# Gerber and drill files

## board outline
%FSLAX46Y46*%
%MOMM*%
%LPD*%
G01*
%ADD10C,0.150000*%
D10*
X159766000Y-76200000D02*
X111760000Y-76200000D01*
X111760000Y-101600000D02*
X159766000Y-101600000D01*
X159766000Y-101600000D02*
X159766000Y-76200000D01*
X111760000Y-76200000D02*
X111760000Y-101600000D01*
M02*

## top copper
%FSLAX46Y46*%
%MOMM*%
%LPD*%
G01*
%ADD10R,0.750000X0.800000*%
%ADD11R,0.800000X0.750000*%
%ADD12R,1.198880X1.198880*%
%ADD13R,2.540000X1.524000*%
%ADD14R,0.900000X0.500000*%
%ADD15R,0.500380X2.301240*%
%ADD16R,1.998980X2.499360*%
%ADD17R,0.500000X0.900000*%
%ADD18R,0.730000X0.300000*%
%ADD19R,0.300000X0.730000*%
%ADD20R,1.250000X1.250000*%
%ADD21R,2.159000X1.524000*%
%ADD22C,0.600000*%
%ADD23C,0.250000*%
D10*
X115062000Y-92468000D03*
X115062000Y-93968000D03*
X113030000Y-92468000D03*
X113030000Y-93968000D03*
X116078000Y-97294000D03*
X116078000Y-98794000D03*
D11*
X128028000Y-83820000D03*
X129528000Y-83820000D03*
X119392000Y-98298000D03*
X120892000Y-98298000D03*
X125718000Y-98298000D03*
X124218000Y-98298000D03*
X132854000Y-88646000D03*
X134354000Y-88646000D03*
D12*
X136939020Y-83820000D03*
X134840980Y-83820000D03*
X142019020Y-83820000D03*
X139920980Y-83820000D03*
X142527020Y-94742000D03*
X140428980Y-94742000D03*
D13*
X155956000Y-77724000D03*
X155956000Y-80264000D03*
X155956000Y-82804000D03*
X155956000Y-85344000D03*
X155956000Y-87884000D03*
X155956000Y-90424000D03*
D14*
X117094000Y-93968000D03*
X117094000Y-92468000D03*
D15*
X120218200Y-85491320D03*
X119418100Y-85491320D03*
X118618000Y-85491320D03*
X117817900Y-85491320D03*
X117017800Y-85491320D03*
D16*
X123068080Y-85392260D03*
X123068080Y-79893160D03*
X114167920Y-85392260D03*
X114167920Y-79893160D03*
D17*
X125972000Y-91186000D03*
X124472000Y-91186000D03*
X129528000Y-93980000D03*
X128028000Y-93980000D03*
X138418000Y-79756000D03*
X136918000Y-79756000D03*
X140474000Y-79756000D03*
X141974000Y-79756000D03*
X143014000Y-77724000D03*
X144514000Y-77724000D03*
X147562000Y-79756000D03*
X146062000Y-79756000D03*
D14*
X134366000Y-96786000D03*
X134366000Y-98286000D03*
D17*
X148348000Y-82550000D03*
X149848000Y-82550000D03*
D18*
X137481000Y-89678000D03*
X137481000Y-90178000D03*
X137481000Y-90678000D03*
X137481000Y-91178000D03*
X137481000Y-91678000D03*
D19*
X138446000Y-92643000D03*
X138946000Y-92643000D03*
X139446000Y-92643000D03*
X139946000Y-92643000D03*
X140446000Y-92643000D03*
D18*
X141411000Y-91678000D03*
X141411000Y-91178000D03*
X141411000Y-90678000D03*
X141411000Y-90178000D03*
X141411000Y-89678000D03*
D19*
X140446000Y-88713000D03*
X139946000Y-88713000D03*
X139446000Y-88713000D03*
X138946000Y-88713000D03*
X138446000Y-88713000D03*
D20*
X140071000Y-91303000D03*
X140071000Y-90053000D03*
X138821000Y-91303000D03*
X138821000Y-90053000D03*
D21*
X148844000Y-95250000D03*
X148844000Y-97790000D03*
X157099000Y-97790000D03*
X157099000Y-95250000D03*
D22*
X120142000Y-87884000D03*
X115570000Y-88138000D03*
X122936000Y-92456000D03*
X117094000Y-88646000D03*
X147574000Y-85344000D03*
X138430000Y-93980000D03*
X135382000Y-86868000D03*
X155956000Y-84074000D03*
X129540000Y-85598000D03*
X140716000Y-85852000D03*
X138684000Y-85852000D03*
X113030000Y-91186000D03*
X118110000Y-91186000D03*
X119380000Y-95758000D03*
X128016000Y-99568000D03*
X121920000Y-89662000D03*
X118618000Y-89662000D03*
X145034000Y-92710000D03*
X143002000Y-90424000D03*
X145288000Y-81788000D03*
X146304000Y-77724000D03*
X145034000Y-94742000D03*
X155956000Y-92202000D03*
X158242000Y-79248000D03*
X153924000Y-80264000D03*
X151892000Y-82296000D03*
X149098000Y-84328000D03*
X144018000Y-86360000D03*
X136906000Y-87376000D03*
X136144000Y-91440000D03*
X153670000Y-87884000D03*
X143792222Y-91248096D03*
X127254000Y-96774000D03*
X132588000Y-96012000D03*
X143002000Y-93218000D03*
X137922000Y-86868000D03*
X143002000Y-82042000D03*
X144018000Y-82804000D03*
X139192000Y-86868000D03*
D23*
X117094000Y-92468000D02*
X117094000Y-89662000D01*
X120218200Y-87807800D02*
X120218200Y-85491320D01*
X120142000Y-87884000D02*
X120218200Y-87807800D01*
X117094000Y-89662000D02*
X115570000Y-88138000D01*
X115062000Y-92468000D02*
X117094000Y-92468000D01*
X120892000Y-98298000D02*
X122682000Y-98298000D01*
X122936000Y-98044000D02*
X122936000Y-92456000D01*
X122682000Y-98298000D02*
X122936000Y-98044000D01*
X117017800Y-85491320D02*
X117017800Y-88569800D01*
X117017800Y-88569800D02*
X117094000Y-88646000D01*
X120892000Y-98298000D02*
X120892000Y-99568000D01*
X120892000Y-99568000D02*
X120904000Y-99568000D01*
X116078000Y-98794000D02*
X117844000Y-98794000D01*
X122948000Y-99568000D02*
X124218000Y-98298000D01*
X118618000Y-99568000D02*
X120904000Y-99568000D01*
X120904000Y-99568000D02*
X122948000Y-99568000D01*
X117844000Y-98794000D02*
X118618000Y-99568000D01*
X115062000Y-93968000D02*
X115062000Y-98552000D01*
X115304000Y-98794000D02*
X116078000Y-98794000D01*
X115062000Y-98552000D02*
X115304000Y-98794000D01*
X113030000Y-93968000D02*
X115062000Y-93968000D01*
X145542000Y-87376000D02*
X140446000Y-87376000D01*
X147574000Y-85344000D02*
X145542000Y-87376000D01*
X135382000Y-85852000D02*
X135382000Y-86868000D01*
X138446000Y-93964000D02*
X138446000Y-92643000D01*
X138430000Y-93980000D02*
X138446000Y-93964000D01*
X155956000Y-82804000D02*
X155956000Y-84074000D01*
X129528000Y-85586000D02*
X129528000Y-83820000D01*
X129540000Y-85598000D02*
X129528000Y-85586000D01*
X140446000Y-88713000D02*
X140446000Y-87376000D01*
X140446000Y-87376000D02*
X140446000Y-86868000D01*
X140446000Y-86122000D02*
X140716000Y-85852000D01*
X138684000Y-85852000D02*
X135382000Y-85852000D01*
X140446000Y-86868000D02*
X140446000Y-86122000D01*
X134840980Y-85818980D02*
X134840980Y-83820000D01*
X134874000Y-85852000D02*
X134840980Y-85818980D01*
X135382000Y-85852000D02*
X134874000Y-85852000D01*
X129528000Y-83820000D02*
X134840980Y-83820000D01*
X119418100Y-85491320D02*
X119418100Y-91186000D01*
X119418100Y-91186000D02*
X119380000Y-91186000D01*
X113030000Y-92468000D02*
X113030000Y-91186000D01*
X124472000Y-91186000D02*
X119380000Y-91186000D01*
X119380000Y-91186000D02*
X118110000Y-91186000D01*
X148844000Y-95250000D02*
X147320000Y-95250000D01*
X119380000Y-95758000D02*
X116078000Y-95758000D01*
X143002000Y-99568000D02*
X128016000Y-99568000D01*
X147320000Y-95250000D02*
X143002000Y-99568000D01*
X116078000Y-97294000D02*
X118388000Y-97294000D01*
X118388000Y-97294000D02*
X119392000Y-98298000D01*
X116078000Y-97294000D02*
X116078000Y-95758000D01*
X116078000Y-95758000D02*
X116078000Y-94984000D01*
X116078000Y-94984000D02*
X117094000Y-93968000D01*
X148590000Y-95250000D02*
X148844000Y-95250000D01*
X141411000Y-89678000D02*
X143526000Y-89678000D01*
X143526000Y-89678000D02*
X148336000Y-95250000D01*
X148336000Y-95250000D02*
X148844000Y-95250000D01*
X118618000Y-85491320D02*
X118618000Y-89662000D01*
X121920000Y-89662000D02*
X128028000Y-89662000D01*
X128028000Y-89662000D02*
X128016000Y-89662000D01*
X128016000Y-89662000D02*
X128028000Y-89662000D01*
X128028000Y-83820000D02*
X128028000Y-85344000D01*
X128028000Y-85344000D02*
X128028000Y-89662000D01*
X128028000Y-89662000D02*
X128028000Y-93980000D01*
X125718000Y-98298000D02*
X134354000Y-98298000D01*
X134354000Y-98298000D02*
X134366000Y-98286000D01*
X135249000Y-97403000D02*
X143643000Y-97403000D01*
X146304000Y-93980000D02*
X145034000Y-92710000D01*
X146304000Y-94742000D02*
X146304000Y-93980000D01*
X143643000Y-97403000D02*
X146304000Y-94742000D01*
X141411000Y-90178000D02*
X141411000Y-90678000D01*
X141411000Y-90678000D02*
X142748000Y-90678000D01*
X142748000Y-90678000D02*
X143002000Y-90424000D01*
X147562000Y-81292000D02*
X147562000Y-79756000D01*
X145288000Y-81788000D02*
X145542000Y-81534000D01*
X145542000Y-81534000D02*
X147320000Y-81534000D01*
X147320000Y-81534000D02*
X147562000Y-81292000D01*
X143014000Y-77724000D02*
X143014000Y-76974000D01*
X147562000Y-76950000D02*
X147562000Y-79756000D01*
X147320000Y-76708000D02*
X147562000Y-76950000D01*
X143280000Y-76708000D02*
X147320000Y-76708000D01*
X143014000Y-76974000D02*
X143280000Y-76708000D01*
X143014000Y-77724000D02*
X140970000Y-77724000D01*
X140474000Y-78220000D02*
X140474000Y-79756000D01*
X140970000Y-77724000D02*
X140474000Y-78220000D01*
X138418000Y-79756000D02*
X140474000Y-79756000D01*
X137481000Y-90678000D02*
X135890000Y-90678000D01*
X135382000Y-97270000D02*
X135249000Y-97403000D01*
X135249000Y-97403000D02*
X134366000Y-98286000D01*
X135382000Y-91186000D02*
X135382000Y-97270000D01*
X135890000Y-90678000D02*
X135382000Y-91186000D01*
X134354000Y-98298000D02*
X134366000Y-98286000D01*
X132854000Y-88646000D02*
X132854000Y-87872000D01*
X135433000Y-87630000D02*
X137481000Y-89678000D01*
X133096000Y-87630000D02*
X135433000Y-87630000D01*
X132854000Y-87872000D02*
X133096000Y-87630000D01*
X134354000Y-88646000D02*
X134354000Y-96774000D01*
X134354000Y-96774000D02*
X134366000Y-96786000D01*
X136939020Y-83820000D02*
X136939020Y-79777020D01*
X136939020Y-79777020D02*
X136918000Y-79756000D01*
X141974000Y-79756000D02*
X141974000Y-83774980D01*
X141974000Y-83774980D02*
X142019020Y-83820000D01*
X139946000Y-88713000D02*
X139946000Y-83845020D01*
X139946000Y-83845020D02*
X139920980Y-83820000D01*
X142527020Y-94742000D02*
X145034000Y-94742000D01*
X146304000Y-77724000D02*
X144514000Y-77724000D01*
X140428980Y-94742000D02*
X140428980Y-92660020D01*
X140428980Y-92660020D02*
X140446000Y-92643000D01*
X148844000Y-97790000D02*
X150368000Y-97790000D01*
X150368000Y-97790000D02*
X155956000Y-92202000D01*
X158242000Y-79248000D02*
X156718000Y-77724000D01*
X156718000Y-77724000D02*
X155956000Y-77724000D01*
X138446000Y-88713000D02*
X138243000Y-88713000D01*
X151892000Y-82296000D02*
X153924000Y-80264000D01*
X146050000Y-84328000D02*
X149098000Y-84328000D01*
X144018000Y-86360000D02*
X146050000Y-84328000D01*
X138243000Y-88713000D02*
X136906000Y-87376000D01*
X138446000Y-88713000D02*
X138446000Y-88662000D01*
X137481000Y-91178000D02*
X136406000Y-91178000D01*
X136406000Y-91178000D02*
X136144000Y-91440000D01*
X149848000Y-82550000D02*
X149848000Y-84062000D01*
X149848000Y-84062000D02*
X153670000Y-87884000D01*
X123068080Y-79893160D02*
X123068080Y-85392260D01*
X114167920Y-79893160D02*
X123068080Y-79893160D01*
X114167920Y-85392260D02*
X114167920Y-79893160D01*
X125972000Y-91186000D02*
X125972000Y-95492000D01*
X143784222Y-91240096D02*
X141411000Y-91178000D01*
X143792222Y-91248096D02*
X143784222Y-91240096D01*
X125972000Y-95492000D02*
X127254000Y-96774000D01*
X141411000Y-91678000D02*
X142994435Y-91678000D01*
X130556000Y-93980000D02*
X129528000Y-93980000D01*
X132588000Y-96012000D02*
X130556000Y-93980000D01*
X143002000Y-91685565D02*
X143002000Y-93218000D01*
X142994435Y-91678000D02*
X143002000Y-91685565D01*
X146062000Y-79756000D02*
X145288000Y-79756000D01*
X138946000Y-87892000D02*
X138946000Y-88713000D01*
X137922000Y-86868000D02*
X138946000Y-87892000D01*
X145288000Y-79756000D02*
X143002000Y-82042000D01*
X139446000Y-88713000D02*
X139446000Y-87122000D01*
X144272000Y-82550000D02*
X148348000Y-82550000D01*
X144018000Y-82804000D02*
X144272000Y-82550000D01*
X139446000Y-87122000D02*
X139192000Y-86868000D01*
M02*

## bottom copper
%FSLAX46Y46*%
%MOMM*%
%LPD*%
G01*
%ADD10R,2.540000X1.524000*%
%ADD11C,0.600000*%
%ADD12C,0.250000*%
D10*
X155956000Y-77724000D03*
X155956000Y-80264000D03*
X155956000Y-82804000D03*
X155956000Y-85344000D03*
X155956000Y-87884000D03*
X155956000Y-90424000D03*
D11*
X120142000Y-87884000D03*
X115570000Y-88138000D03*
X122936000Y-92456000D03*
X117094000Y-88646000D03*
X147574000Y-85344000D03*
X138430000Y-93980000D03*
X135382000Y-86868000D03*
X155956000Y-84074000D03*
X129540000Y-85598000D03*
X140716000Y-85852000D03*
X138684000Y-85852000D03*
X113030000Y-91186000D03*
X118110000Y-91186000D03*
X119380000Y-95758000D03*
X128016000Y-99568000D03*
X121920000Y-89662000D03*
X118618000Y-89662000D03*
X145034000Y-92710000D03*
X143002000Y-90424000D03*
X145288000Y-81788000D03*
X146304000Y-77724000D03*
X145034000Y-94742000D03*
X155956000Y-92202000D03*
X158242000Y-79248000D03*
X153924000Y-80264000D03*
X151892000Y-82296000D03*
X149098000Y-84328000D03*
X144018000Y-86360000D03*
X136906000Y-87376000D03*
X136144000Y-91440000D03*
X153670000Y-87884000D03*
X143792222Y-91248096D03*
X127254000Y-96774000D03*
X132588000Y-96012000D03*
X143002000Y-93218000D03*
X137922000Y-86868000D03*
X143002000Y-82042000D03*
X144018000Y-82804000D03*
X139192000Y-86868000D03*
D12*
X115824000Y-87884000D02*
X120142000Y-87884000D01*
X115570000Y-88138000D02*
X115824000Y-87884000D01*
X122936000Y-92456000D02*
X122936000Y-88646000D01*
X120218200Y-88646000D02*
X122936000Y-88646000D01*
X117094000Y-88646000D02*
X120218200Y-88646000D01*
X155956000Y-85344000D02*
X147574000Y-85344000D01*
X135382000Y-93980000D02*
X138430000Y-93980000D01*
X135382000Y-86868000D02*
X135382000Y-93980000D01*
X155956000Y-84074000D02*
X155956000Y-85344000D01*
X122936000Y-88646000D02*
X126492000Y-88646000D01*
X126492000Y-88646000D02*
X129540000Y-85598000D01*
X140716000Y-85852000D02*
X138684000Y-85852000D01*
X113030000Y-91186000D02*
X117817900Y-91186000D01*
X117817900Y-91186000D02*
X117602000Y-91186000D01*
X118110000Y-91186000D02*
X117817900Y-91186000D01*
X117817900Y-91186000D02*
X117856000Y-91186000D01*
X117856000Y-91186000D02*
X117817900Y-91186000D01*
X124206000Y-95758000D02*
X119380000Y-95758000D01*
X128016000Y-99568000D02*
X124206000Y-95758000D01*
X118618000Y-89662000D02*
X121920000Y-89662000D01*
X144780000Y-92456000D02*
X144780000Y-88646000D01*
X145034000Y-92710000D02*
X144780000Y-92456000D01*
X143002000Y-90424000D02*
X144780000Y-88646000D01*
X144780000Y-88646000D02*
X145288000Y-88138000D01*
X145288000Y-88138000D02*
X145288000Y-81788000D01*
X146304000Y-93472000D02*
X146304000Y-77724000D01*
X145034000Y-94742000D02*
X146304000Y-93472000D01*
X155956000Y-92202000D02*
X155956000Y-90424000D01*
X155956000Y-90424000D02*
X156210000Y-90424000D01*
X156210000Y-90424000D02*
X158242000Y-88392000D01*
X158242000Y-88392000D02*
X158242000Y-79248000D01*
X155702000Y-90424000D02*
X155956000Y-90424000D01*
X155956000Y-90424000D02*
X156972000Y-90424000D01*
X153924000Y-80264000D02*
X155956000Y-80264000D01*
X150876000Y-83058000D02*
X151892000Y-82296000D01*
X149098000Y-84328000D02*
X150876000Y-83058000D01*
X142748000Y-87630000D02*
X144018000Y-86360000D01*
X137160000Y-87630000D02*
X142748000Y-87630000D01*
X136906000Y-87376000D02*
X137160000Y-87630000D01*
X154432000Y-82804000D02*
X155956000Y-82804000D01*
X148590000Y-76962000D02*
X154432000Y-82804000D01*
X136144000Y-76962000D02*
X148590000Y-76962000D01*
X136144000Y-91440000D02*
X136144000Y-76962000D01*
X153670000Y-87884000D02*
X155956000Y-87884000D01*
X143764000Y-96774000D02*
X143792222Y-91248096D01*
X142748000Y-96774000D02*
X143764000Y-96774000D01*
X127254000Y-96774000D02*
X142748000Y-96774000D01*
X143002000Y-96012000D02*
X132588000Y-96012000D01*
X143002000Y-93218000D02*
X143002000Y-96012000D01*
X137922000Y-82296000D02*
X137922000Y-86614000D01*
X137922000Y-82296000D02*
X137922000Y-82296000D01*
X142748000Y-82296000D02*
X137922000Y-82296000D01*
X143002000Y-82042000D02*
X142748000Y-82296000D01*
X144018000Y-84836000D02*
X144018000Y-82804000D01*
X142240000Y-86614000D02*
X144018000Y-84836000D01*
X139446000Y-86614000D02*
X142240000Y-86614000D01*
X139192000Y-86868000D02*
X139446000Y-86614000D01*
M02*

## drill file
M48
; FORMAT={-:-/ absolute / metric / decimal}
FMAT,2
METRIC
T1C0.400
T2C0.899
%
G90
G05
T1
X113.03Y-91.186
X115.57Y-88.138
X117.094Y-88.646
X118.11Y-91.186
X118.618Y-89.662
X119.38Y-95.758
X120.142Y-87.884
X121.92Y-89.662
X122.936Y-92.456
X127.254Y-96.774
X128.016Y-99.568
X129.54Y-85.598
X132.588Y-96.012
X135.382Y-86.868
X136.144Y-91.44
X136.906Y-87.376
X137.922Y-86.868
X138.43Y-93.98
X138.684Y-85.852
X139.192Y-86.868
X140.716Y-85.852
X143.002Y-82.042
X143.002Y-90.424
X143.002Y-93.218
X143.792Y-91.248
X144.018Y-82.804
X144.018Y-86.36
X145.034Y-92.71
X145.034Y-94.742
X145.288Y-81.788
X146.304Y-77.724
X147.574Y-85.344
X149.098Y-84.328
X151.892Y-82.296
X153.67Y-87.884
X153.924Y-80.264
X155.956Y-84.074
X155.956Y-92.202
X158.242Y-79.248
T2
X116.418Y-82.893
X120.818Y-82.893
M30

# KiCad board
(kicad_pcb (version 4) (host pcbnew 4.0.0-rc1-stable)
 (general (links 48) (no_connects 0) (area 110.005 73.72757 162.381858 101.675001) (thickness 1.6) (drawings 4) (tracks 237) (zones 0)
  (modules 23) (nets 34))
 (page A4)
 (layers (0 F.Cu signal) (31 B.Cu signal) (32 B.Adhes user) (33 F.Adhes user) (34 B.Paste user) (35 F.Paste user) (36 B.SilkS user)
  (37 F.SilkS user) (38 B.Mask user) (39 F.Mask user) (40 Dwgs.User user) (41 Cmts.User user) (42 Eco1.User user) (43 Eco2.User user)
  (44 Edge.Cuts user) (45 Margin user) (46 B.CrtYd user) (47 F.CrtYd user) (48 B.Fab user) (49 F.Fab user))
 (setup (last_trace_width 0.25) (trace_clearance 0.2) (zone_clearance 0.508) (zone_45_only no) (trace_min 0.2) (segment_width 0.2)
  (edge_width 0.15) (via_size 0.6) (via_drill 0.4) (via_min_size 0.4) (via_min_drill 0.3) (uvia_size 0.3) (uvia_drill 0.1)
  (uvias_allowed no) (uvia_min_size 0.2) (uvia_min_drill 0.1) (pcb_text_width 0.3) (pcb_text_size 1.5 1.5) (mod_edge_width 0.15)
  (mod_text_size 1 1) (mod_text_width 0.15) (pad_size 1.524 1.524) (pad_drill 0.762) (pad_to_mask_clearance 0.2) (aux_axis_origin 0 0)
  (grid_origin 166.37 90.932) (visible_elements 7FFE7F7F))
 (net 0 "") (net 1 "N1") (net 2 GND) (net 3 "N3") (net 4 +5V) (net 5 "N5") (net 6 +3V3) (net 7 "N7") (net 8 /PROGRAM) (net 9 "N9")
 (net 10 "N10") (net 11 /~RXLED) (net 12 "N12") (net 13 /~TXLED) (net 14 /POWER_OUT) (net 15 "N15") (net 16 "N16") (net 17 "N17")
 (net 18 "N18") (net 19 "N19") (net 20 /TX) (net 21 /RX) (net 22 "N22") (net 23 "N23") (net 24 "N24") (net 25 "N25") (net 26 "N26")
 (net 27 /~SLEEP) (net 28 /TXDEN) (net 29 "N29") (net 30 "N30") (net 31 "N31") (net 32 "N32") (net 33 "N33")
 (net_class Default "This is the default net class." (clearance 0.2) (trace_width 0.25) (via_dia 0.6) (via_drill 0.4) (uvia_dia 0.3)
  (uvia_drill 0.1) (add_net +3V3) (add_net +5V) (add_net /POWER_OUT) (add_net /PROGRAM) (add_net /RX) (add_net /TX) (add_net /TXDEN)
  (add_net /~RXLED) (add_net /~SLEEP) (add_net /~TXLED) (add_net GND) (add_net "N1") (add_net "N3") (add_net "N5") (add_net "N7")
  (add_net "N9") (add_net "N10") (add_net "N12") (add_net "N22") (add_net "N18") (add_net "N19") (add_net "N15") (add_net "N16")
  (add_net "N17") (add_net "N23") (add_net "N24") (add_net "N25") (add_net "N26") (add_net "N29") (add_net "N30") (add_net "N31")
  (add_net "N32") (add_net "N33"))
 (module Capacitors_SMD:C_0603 (layer F.Cu) (at 115.062 93.218 270)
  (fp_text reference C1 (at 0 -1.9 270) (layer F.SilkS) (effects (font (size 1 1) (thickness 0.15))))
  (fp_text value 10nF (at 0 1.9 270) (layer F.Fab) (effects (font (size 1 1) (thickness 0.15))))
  (pad 1 smd rect (at -0.75 0 270) (size 0.8 0.75) (layers F.Cu F.Paste F.Mask) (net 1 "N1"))
  (pad 2 smd rect (at 0.75 0 270) (size 0.8 0.75) (layers F.Cu F.Paste F.Mask) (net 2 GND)))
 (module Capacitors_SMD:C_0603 (layer F.Cu) (at 113.03 93.218 270)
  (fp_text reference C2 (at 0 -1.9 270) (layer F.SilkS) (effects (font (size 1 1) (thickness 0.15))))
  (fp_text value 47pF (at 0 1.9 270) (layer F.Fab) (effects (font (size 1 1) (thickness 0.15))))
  (pad 1 smd rect (at -0.75 0 270) (size 0.8 0.75) (layers F.Cu F.Paste F.Mask) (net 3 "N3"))
  (pad 2 smd rect (at 0.75 0 270) (size 0.8 0.75) (layers F.Cu F.Paste F.Mask) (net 2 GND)))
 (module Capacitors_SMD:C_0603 (layer F.Cu) (at 116.078 98.044 270)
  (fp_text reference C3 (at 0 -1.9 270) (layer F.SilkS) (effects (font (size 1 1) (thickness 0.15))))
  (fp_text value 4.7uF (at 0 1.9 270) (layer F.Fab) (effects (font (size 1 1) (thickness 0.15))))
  (pad 1 smd rect (at -0.75 0 270) (size 0.8 0.75) (layers F.Cu F.Paste F.Mask) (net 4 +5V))
  (pad 2 smd rect (at 0.75 0 270) (size 0.8 0.75) (layers F.Cu F.Paste F.Mask) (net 2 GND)))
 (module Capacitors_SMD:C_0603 (layer F.Cu) (at 128.778 83.82)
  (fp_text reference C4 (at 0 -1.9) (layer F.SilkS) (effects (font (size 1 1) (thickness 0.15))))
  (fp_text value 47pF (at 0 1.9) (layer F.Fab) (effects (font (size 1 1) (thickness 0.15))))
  (pad 1 smd rect (at -0.75 0) (size 0.8 0.75) (layers F.Cu F.Paste F.Mask) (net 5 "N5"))
  (pad 2 smd rect (at 0.75 0) (size 0.8 0.75) (layers F.Cu F.Paste F.Mask) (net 2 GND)))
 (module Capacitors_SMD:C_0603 (layer F.Cu) (at 120.142 98.298)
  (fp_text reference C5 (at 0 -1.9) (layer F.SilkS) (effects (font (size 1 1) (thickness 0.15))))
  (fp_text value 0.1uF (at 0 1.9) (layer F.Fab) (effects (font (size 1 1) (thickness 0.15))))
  (pad 1 smd rect (at -0.75 0) (size 0.8 0.75) (layers F.Cu F.Paste F.Mask) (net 4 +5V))
  (pad 2 smd rect (at 0.75 0) (size 0.8 0.75) (layers F.Cu F.Paste F.Mask) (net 2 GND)))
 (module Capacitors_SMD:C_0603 (layer F.Cu) (at 124.968 98.298 180)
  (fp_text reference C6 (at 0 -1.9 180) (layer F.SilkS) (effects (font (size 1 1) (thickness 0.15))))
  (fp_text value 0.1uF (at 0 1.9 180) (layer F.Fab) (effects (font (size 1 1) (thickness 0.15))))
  (pad 1 smd rect (at -0.75 0 180) (size 0.8 0.75) (layers F.Cu F.Paste F.Mask) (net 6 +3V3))
  (pad 2 smd rect (at 0.75 0 180) (size 0.8 0.75) (layers F.Cu F.Paste F.Mask) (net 2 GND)))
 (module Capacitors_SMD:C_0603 (layer F.Cu) (at 133.604 88.646)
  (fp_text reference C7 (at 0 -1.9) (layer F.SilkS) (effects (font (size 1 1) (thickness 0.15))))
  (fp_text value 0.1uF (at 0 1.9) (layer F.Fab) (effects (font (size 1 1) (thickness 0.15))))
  (pad 1 smd rect (at -0.75 0) (size 0.8 0.75) (layers F.Cu F.Paste F.Mask) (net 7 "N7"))
  (pad 2 smd rect (at 0.75 0) (size 0.8 0.75) (layers F.Cu F.Paste F.Mask) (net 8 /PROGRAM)))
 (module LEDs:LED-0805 (layer F.Cu) (at 135.89 83.82)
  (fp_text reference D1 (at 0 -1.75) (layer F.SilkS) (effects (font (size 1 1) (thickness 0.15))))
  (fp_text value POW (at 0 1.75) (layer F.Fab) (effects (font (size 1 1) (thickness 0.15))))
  (pad 2 smd rect (at 1.04902 0 180) (size 1.19888 1.19888) (layers F.Cu F.Paste F.Mask) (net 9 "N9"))
  (pad 1 smd rect (at -1.04902 0 180) (size 1.19888 1.19888) (layers F.Cu F.Paste F.Mask) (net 2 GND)))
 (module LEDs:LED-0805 (layer F.Cu) (at 140.97 83.82)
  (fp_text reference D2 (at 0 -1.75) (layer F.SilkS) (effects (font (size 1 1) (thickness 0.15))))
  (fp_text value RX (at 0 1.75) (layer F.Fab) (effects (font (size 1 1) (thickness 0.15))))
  (pad 2 smd rect (at 1.04902 0 180) (size 1.19888 1.19888) (layers F.Cu F.Paste F.Mask) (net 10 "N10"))
  (pad 1 smd rect (at -1.04902 0 180) (size 1.19888 1.19888) (layers F.Cu F.Paste F.Mask) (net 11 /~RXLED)))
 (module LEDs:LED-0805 (layer F.Cu) (at 141.478 94.742)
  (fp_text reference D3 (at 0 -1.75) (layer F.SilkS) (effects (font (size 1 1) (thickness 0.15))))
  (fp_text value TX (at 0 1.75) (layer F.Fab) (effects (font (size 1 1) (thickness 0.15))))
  (pad 2 smd rect (at 1.04902 0 180) (size 1.19888 1.19888) (layers F.Cu F.Paste F.Mask) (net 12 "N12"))
  (pad 1 smd rect (at -1.04902 0 180) (size 1.19888 1.19888) (layers F.Cu F.Paste F.Mask) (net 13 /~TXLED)))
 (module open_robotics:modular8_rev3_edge (layer F.Cu) (at 155.956 82.804 270)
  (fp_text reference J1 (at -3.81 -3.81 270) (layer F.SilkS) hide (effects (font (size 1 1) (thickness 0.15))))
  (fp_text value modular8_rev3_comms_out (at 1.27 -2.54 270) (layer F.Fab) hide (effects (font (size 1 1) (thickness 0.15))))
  (pad 1 smd rect (at -5.08 0 270) (size 1.524 2.54) (layers F.Cu F.Paste F.Mask) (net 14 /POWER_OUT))
  (pad 3 smd rect (at -2.54 0 270) (size 1.524 2.54) (layers F.Cu F.Paste F.Mask) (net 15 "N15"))
  (pad 5 smd rect (at 0 0 270) (size 1.524 2.54) (layers F.Cu F.Paste F.Mask) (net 2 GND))
  (pad 7 smd rect (at 2.54 0 270) (size 1.524 2.54) (layers F.Cu F.Paste F.Mask) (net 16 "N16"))
  (pad 9 smd rect (at 5.08 0 270) (size 1.524 2.54) (layers F.Cu F.Paste F.Mask) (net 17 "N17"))
  (pad 11 smd rect (at 7.62 0 270) (size 1.524 2.54) (layers F.Cu F.Paste F.Mask) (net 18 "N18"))
  (pad 2 smd rect (at -5.08 0 270) (size 1.524 2.54) (layers B.Cu F.Paste F.Mask) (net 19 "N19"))
  (pad 4 smd rect (at -2.54 0 270) (size 1.524 2.54) (layers B.Cu F.Paste F.Mask) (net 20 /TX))
  (pad 6 smd rect (at 0 0 270) (size 1.524 2.54) (layers B.Cu F.Paste F.Mask) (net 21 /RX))
  (pad 8 smd rect (at 2.54 0 270) (size 1.524 2.54) (layers B.Cu F.Paste F.Mask) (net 2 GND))
  (pad 10 smd rect (at 5.08 0 270) (size 1.524 2.54) (layers B.Cu F.Paste F.Mask) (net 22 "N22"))
  (pad 12 smd rect (at 7.62 0 270) (size 1.524 2.54) (layers B.Cu F.Paste F.Mask) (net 14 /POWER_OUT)))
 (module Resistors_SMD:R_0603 (layer F.Cu) (at 117.094 93.218 90)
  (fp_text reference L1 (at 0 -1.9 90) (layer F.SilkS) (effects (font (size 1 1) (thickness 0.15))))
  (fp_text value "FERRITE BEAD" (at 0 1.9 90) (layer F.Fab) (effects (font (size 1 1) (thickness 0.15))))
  (pad 1 smd rect (at -0.75 0 90) (size 0.5 0.9) (layers F.Cu F.Paste F.Mask) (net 4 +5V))
  (pad 2 smd rect (at 0.75 0 90) (size 0.5 0.9) (layers F.Cu F.Paste F.Mask) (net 1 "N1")))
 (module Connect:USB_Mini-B (layer F.Cu) (at 118.618 82.042 270)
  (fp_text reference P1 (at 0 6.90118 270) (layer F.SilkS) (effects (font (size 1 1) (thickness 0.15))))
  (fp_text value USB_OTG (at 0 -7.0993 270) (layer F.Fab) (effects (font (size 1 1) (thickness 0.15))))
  (pad 1 smd rect (at 3.44932 -1.6002 270) (size 2.30124 0.50038) (layers F.Cu F.Paste F.Mask) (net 1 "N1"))
  (pad 2 smd rect (at 3.44932 -0.8001 270) (size 2.30124 0.50038) (layers F.Cu F.Paste F.Mask) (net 3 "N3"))
  (pad 3 smd rect (at 3.44932 0 270) (size 2.30124 0.50038) (layers F.Cu F.Paste F.Mask) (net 5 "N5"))
  (pad 4 smd rect (at 3.44932 0.8001 270) (size 2.30124 0.50038) (layers F.Cu F.Paste F.Mask) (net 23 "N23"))
  (pad 5 smd rect (at 3.44932 1.6002 270) (size 2.30124 0.50038) (layers F.Cu F.Paste F.Mask) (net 2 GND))
  (pad 6 smd rect (at 3.35026 -4.45008 270) (size 2.49936 1.99898) (layers F.Cu F.Paste F.Mask) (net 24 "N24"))
  (pad 6 smd rect (at -2.14884 -4.45008 270) (size 2.49936 1.99898) (layers F.Cu F.Paste F.Mask) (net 24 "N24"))
  (pad 6 smd rect (at 3.35026 4.45008 270) (size 2.49936 1.99898) (layers F.Cu F.Paste F.Mask) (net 24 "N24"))
  (pad 6 smd rect (at -2.14884 4.45008 270) (size 2.49936 1.99898) (layers F.Cu F.Paste F.Mask) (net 24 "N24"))
  (pad "" np_thru_hole circle (at 0.8509 -2.19964 270) (size 0.89916 0.89916) (drill 0.89916) (layers *.Cu *.Mask F.SilkS))
  (pad "" np_thru_hole circle (at 0.8509 2.19964 270) (size 0.89916 0.89916) (drill 0.89916) (layers *.Cu *.Mask F.SilkS)))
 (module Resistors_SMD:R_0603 (layer F.Cu) (at 125.222 91.186 180)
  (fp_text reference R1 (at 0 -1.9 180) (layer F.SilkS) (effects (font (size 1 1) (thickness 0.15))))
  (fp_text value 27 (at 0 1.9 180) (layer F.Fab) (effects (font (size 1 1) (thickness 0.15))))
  (pad 1 smd rect (at -0.75 0 180) (size 0.5 0.9) (layers F.Cu F.Paste F.Mask) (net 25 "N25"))
  (pad 2 smd rect (at 0.75 0 180) (size 0.5 0.9) (layers F.Cu F.Paste F.Mask) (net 3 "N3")))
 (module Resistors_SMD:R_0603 (layer F.Cu) (at 128.778 93.98 180)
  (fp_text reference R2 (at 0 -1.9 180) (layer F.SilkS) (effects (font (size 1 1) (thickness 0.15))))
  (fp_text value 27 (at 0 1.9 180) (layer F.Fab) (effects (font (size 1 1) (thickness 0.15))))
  (pad 1 smd rect (at -0.75 0 180) (size 0.5 0.9) (layers F.Cu F.Paste F.Mask) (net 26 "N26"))
  (pad 2 smd rect (at 0.75 0 180) (size 0.5 0.9) (layers F.Cu F.Paste F.Mask) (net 5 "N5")))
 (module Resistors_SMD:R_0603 (layer F.Cu) (at 137.668 79.756 180)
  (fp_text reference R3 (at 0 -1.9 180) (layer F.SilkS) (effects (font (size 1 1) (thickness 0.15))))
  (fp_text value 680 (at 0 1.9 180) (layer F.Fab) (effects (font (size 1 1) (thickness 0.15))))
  (pad 1 smd rect (at -0.75 0 180) (size 0.5 0.9) (layers F.Cu F.Paste F.Mask) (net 6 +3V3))
  (pad 2 smd rect (at 0.75 0 180) (size 0.5 0.9) (layers F.Cu F.Paste F.Mask) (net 9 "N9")))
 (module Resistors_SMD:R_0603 (layer F.Cu) (at 141.224 79.756)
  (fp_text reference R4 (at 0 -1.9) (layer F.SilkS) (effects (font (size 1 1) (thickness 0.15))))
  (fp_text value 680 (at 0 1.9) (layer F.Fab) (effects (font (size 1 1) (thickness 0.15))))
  (pad 1 smd rect (at -0.75 0) (size 0.5 0.9) (layers F.Cu F.Paste F.Mask) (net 6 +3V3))
  (pad 2 smd rect (at 0.75 0) (size 0.5 0.9) (layers F.Cu F.Paste F.Mask) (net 10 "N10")))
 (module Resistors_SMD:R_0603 (layer F.Cu) (at 143.764 77.724)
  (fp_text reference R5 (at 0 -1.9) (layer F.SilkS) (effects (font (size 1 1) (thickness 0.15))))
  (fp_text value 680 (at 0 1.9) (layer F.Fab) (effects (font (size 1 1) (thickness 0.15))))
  (pad 1 smd rect (at -0.75 0) (size 0.5 0.9) (layers F.Cu F.Paste F.Mask) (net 6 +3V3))
  (pad 2 smd rect (at 0.75 0) (size 0.5 0.9) (layers F.Cu F.Paste F.Mask) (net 12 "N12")))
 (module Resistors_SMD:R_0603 (layer F.Cu) (at 146.812 79.756 180)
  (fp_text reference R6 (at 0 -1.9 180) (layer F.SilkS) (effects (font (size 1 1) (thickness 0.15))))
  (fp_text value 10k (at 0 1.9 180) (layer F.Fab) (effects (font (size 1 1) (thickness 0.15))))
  (pad 1 smd rect (at -0.75 0 180) (size 0.5 0.9) (layers F.Cu F.Paste F.Mask) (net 6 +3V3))
  (pad 2 smd rect (at 0.75 0 180) (size 0.5 0.9) (layers F.Cu F.Paste F.Mask) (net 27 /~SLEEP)))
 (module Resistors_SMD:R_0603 (layer F.Cu) (at 134.366 97.536 270)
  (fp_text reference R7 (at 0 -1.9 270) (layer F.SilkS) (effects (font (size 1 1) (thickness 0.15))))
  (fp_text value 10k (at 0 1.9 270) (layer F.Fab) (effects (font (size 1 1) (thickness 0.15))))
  (pad 1 smd rect (at -0.75 0 270) (size 0.5 0.9) (layers F.Cu F.Paste F.Mask) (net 8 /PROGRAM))
  (pad 2 smd rect (at 0.75 0 270) (size 0.5 0.9) (layers F.Cu F.Paste F.Mask) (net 6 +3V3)))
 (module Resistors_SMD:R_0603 (layer F.Cu) (at 149.098 82.55)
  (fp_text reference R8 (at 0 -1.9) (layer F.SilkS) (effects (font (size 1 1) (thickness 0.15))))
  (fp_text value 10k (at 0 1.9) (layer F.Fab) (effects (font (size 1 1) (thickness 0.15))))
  (pad 1 smd rect (at -0.75 0) (size 0.5 0.9) (layers F.Cu F.Paste F.Mask) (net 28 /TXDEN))
  (pad 2 smd rect (at 0.75 0) (size 0.5 0.9) (layers F.Cu F.Paste F.Mask) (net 22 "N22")))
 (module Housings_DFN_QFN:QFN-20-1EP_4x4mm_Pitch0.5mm (layer F.Cu) (at 139.446 90.678)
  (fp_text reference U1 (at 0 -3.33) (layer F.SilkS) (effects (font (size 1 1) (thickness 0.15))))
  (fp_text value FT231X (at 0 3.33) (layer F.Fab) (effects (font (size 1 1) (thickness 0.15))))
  (pad 1 smd rect (at -1.965 -1) (size 0.73 0.3) (layers F.Cu F.Paste F.Mask) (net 7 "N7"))
  (pad 2 smd rect (at -1.965 -0.5) (size 0.73 0.3) (layers F.Cu F.Paste F.Mask) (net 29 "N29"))
  (pad 3 smd rect (at -1.965 0) (size 0.73 0.3) (layers F.Cu F.Paste F.Mask) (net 6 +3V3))
  (pad 4 smd rect (at -1.965 0.5) (size 0.73 0.3) (layers F.Cu F.Paste F.Mask) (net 21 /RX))
  (pad 5 smd rect (at -1.965 1) (size 0.73 0.3) (layers F.Cu F.Paste F.Mask) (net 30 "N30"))
  (pad 6 smd rect (at -1 1.965 90) (size 0.73 0.3) (layers F.Cu F.Paste F.Mask) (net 2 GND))
  (pad 7 smd rect (at -0.5 1.965 90) (size 0.73 0.3) (layers F.Cu F.Paste F.Mask) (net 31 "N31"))
  (pad 8 smd rect (at 0 1.965 90) (size 0.73 0.3) (layers F.Cu F.Paste F.Mask) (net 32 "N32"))
  (pad 9 smd rect (at 0.5 1.965 90) (size 0.73 0.3) (layers F.Cu F.Paste F.Mask) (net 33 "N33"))
  (pad 10 smd rect (at 1 1.965 90) (size 0.73 0.3) (layers F.Cu F.Paste F.Mask) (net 13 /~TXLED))
  (pad 11 smd rect (at 1.965 1) (size 0.73 0.3) (layers F.Cu F.Paste F.Mask) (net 26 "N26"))
  (pad 12 smd rect (at 1.965 0.5) (size 0.73 0.3) (layers F.Cu F.Paste F.Mask) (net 25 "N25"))
  (pad 13 smd rect (at 1.965 0) (size 0.73 0.3) (layers F.Cu F.Paste F.Mask) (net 6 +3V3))
  (pad 14 smd rect (at 1.965 -0.5) (size 0.73 0.3) (layers F.Cu F.Paste F.Mask) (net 6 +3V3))
  (pad 15 smd rect (at 1.965 -1) (size 0.73 0.3) (layers F.Cu F.Paste F.Mask) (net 4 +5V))
  (pad 16 smd rect (at 1 -1.965 90) (size 0.73 0.3) (layers F.Cu F.Paste F.Mask) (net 2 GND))
  (pad 17 smd rect (at 0.5 -1.965 90) (size 0.73 0.3) (layers F.Cu F.Paste F.Mask) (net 11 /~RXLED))
  (pad 18 smd rect (at 0 -1.965 90) (size 0.73 0.3) (layers F.Cu F.Paste F.Mask) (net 28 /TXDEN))
  (pad 19 smd rect (at -0.5 -1.965 90) (size 0.73 0.3) (layers F.Cu F.Paste F.Mask) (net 27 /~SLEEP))
  (pad 20 smd rect (at -1 -1.965 90) (size 0.73 0.3) (layers F.Cu F.Paste F.Mask) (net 20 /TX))
  (pad 21 smd rect (at 0.625 0.625) (size 1.25 1.25) (layers F.Cu F.Paste F.Mask) (solder_paste_margin_ratio -0.2))
  (pad 21 smd rect (at 0.625 -0.625) (size 1.25 1.25) (layers F.Cu F.Paste F.Mask) (solder_paste_margin_ratio -0.2))
  (pad 21 smd rect (at -0.625 0.625) (size 1.25 1.25) (layers F.Cu F.Paste F.Mask) (solder_paste_margin_ratio -0.2))
  (pad 21 smd rect (at -0.625 -0.625) (size 1.25 1.25) (layers F.Cu F.Paste F.Mask) (solder_paste_margin_ratio -0.2)))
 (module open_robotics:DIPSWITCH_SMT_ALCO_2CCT (layer F.Cu) (at 148.844 95.25)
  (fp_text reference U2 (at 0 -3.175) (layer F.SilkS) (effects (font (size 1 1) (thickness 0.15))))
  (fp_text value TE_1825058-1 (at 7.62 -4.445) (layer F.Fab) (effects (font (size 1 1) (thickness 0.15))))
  (pad 1 smd rect (at 0 0) (size 2.159 1.524) (layers F.Cu F.Paste F.Mask) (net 4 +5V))
  (pad 2 smd rect (at 0 2.54) (size 2.159 1.524) (layers F.Cu F.Paste F.Mask) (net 14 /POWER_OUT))
  (pad 3 smd rect (at 8.255 2.54) (size 2.159 1.524) (layers F.Cu F.Paste F.Mask))
  (pad 4 smd rect (at 8.255 0) (size 2.159 1.524) (layers F.Cu F.Paste F.Mask)))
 (gr_line (start 159.766 76.2) (end 111.76 76.2) (angle 90) (layer Edge.Cuts) (width 0.15))
 (gr_line (start 111.76 101.6) (end 159.766 101.6) (angle 90) (layer Edge.Cuts) (width 0.15))
 (gr_line (start 159.766 101.6) (end 159.766 76.2) (angle 90) (layer Edge.Cuts) (width 0.15))
 (gr_line (start 111.76 76.2) (end 111.76 101.6) (angle 90) (layer Edge.Cuts) (width 0.15))
 (segment (start 117.094 92.468) (end 117.094 89.662) (width 0.25) (layer F.Cu) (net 1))
 (segment (start 120.2182 87.8078) (end 120.2182 85.49132) (width 0.25) (layer F.Cu) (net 1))
 (segment (start 120.142 87.884) (end 120.2182 87.8078) (width 0.25) (layer F.Cu) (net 1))
 (via (at 120.142 87.884) (size 0.6) (drill 0.4) (layers F.Cu B.Cu) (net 1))
 (segment (start 115.824 87.884) (end 120.142 87.884) (width 0.25) (layer B.Cu) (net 1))
 (segment (start 115.57 88.138) (end 115.824 87.884) (width 0.25) (layer B.Cu) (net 1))
 (via (at 115.57 88.138) (size 0.6) (drill 0.4) (layers F.Cu B.Cu) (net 1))
 (segment (start 117.094 89.662) (end 115.57 88.138) (width 0.25) (layer F.Cu) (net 1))
 (segment (start 115.062 92.468) (end 117.094 92.468) (width 0.25) (layer F.Cu) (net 1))
 (segment (start 120.892 98.298) (end 122.682 98.298) (width 0.25) (layer F.Cu) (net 2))
 (segment (start 122.936 92.456) (end 122.936 88.646) (width 0.25) (layer B.Cu) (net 2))
 (via (at 122.936 92.456) (size 0.6) (drill 0.4) (layers F.Cu B.Cu) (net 2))
 (segment (start 122.936 98.044) (end 122.936 92.456) (width 0.25) (layer F.Cu) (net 2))
 (segment (start 122.682 98.298) (end 122.936 98.044) (width 0.25) (layer F.Cu) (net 2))
 (segment (start 117.0178 85.49132) (end 117.0178 88.5698) (width 0.25) (layer F.Cu) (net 2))
 (segment (start 120.2182 88.646) (end 122.936 88.646) (width 0.25) (layer B.Cu) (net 2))
 (segment (start 117.0178 88.5698) (end 117.094 88.646) (width 0.25) (layer F.Cu) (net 2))
 (via (at 117.094 88.646) (size 0.6) (drill 0.4) (layers F.Cu B.Cu) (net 2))
 (segment (start 117.094 88.646) (end 120.2182 88.646) (width 0.25) (layer B.Cu) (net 2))
 (segment (start 120.892 98.298) (end 120.892 99.568) (width 0.25) (layer F.Cu) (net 2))
 (segment (start 120.892 99.568) (end 120.904 99.568) (width 0.25) (layer F.Cu) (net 2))
 (segment (start 116.078 98.794) (end 117.844 98.794) (width 0.25) (layer F.Cu) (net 2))
 (segment (start 122.948 99.568) (end 124.218 98.298) (width 0.25) (layer F.Cu) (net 2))
 (segment (start 118.618 99.568) (end 120.904 99.568) (width 0.25) (layer F.Cu) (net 2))
 (segment (start 120.904 99.568) (end 122.948 99.568) (width 0.25) (layer F.Cu) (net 2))
 (segment (start 117.844 98.794) (end 118.618 99.568) (width 0.25) (layer F.Cu) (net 2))
 (segment (start 115.062 93.968) (end 115.062 98.552) (width 0.25) (layer F.Cu) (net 2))
 (segment (start 115.304 98.794) (end 116.078 98.794) (width 0.25) (layer F.Cu) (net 2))
 (segment (start 115.062 98.552) (end 115.304 98.794) (width 0.25) (layer F.Cu) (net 2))
 (segment (start 113.03 93.968) (end 115.062 93.968) (width 0.25) (layer F.Cu) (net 2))
 (segment (start 155.956 85.344) (end 147.574 85.344) (width 0.25) (layer B.Cu) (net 2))
 (segment (start 145.542 87.376) (end 140.446 87.376) (width 0.25) (layer F.Cu) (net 2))
 (segment (start 147.574 85.344) (end 145.542 87.376) (width 0.25) (layer F.Cu) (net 2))
 (via (at 147.574 85.344) (size 0.6) (drill 0.4) (layers F.Cu B.Cu) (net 2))
 (segment (start 135.382 85.852) (end 135.382 86.868) (width 0.25) (layer F.Cu) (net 2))
 (segment (start 138.446 93.964) (end 138.446 92.643) (width 0.25) (layer F.Cu) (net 2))
 (segment (start 138.43 93.98) (end 138.446 93.964) (width 0.25) (layer F.Cu) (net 2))
 (via (at 138.43 93.98) (size 0.6) (drill 0.4) (layers F.Cu B.Cu) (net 2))
 (segment (start 135.382 93.98) (end 138.43 93.98) (width 0.25) (layer B.Cu) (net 2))
 (segment (start 135.382 86.868) (end 135.382 93.98) (width 0.25) (layer B.Cu) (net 2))
 (via (at 135.382 86.868) (size 0.6) (drill 0.4) (layers F.Cu B.Cu) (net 2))
 (segment (start 155.956 82.804) (end 155.956 84.074) (width 0.25) (layer F.Cu) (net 2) (status 10))
 (segment (start 155.956 84.074) (end 155.956 85.344) (width 0.25) (layer B.Cu) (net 2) (status 20))
 (via (at 155.956 84.074) (size 0.6) (drill 0.4) (layers F.Cu B.Cu) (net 2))
 (segment (start 122.936 88.646) (end 126.492 88.646) (width 0.25) (layer B.Cu) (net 2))
 (segment (start 129.528 85.586) (end 129.528 83.82) (width 0.25) (layer F.Cu) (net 2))
 (segment (start 129.54 85.598) (end 129.528 85.586) (width 0.25) (layer F.Cu) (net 2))
 (via (at 129.54 85.598) (size 0.6) (drill 0.4) (layers F.Cu B.Cu) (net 2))
 (segment (start 126.492 88.646) (end 129.54 85.598) (width 0.25) (layer B.Cu) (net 2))
 (segment (start 140.446 88.713) (end 140.446 87.376) (width 0.25) (layer F.Cu) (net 2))
 (segment (start 140.446 87.376) (end 140.446 86.868) (width 0.25) (layer F.Cu) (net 2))
 (segment (start 140.446 86.122) (end 140.716 85.852) (width 0.25) (layer F.Cu) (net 2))
 (via (at 140.716 85.852) (size 0.6) (drill 0.4) (layers F.Cu B.Cu) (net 2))
 (segment (start 140.716 85.852) (end 138.684 85.852) (width 0.25) (layer B.Cu) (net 2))
 (via (at 138.684 85.852) (size 0.6) (drill 0.4) (layers F.Cu B.Cu) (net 2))
 (segment (start 138.684 85.852) (end 135.382 85.852) (width 0.25) (layer F.Cu) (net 2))
 (segment (start 140.446 86.868) (end 140.446 86.122) (width 0.25) (layer F.Cu) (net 2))
 (segment (start 134.84098 85.81898) (end 134.84098 83.82) (width 0.25) (layer F.Cu) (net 2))
 (segment (start 134.874 85.852) (end 134.84098 85.81898) (width 0.25) (layer F.Cu) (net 2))
 (segment (start 135.382 85.852) (end 134.874 85.852) (width 0.25) (layer F.Cu) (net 2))
 (segment (start 129.528 83.82) (end 134.84098 83.82) (width 0.25) (layer F.Cu) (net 2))
 (segment (start 119.4181 85.49132) (end 119.4181 91.186) (width 0.25) (layer F.Cu) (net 3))
 (segment (start 119.4181 91.186) (end 119.38 91.186) (width 0.25) (layer F.Cu) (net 3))
 (segment (start 113.03 92.468) (end 113.03 91.186) (width 0.25) (layer F.Cu) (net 3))
 (segment (start 113.03 91.186) (end 117.8179 91.186) (width 0.25) (layer B.Cu) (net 3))
 (via (at 113.03 91.186) (size 0.6) (drill 0.4) (layers F.Cu B.Cu) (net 3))
 (segment (start 117.8179 91.186) (end 117.602 91.186) (width 0.25) (layer B.Cu) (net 3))
 (segment (start 124.472 91.186) (end 119.38 91.186) (width 0.25) (layer F.Cu) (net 3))
 (segment (start 119.38 91.186) (end 118.11 91.186) (width 0.25) (layer F.Cu) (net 3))
 (segment (start 118.11 91.186) (end 117.8179 91.186) (width 0.25) (layer B.Cu) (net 3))
 (via (at 118.11 91.186) (size 0.6) (drill 0.4) (layers F.Cu B.Cu) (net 3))
 (segment (start 117.8179 91.186) (end 117.856 91.186) (width 0.25) (layer B.Cu) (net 3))
 (segment (start 117.856 91.186) (end 117.8179 91.186) (width 0.25) (layer B.Cu) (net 3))
 (segment (start 148.844 95.25) (end 147.32 95.25) (width 0.25) (layer F.Cu) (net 4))
 (segment (start 119.38 95.758) (end 116.078 95.758) (width 0.25) (layer F.Cu) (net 4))
 (via (at 119.38 95.758) (size 0.6) (drill 0.4) (layers F.Cu B.Cu) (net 4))
 (segment (start 124.206 95.758) (end 119.38 95.758) (width 0.25) (layer B.Cu) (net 4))
 (segment (start 128.016 99.568) (end 124.206 95.758) (width 0.25) (layer B.Cu) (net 4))
 (via (at 128.016 99.568) (size 0.6) (drill 0.4) (layers F.Cu B.Cu) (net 4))
 (segment (start 143.002 99.568) (end 128.016 99.568) (width 0.25) (layer F.Cu) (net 4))
 (segment (start 147.32 95.25) (end 143.002 99.568) (width 0.25) (layer F.Cu) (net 4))
 (segment (start 116.078 97.294) (end 118.388 97.294) (width 0.25) (layer F.Cu) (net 4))
 (segment (start 118.388 97.294) (end 119.392 98.298) (width 0.25) (layer F.Cu) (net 4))
 (segment (start 116.078 97.294) (end 116.078 95.758) (width 0.25) (layer F.Cu) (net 4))
 (segment (start 116.078 95.758) (end 116.078 94.984) (width 0.25) (layer F.Cu) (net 4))
 (segment (start 116.078 94.984) (end 117.094 93.968) (width 0.25) (layer F.Cu) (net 4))
 (segment (start 148.59 95.25) (end 148.844 95.25) (width 0.25) (layer F.Cu) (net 4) (status 30))
 (segment (start 141.411 89.678) (end 143.526 89.678) (width 0.25) (layer F.Cu) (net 4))
 (segment (start 143.526 89.678) (end 148.336 95.25) (width 0.25) (layer F.Cu) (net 4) (status 20))
 (segment (start 148.336 95.25) (end 148.844 95.25) (width 0.25) (layer F.Cu) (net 4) (status 30))
 (segment (start 118.618 85.49132) (end 118.618 89.662) (width 0.25) (layer F.Cu) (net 5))
 (segment (start 121.92 89.662) (end 128.028 89.662) (width 0.25) (layer F.Cu) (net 5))
 (via (at 121.92 89.662) (size 0.6) (drill 0.4) (layers F.Cu B.Cu) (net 5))
 (segment (start 118.618 89.662) (end 121.92 89.662) (width 0.25) (layer B.Cu) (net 5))
 (via (at 118.618 89.662) (size 0.6) (drill 0.4) (layers F.Cu B.Cu) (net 5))
 (segment (start 128.028 89.662) (end 128.016 89.662) (width 0.25) (layer F.Cu) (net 5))
 (segment (start 128.016 89.662) (end 128.028 89.662) (width 0.25) (layer F.Cu) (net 5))
 (segment (start 128.028 83.82) (end 128.028 85.344) (width 0.25) (layer F.Cu) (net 5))
 (segment (start 128.028 85.344) (end 128.028 89.662) (width 0.25) (layer F.Cu) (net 5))
 (segment (start 128.028 89.662) (end 128.028 93.98) (width 0.25) (layer F.Cu) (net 5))
 (segment (start 125.718 98.298) (end 134.354 98.298) (width 0.25) (layer F.Cu) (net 6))
 (segment (start 134.354 98.298) (end 134.366 98.286) (width 0.25) (layer F.Cu) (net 6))
 (segment (start 135.249 97.403) (end 143.643 97.403) (width 0.25) (layer F.Cu) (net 6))
 (segment (start 144.78 92.456) (end 144.78 88.646) (width 0.25) (layer B.Cu) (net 6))
 (segment (start 145.034 92.71) (end 144.78 92.456) (width 0.25) (layer B.Cu) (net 6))
 (via (at 145.034 92.71) (size 0.6) (drill 0.4) (layers F.Cu B.Cu) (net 6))
 (segment (start 146.304 93.98) (end 145.034 92.71) (width 0.25) (layer F.Cu) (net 6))
 (segment (start 146.304 94.742) (end 146.304 93.98) (width 0.25) (layer F.Cu) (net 6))
 (segment (start 143.643 97.403) (end 146.304 94.742) (width 0.25) (layer F.Cu) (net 6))
 (segment (start 141.411 90.178) (end 141.411 90.678) (width 0.25) (layer F.Cu) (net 6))
 (segment (start 141.411 90.678) (end 142.748 90.678) (width 0.25) (layer F.Cu) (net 6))
 (segment (start 142.748 90.678) (end 143.002 90.424) (width 0.25) (layer F.Cu) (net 6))
 (via (at 143.002 90.424) (size 0.6) (drill 0.4) (layers F.Cu B.Cu) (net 6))
 (segment (start 143.002 90.424) (end 144.78 88.646) (width 0.25) (layer B.Cu) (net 6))
 (segment (start 147.562 81.292) (end 147.562 79.756) (width 0.25) (layer F.Cu) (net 6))
 (segment (start 144.78 88.646) (end 145.288 88.138) (width 0.25) (layer B.Cu) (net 6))
 (segment (start 145.288 88.138) (end 145.288 81.788) (width 0.25) (layer B.Cu) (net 6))
 (via (at 145.288 81.788) (size 0.6) (drill 0.4) (layers F.Cu B.Cu) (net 6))
 (segment (start 145.288 81.788) (end 145.542 81.534) (width 0.25) (layer F.Cu) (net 6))
 (segment (start 145.542 81.534) (end 147.32 81.534) (width 0.25) (layer F.Cu) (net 6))
 (segment (start 147.32 81.534) (end 147.562 81.292) (width 0.25) (layer F.Cu) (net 6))
 (segment (start 143.014 77.724) (end 143.014 76.974) (width 0.25) (layer F.Cu) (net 6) (status 10))
 (segment (start 147.562 76.95) (end 147.562 79.756) (width 0.25) (layer F.Cu) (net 6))
 (segment (start 147.32 76.708) (end 147.562 76.95) (width 0.25) (layer F.Cu) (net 6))
 (segment (start 143.28 76.708) (end 147.32 76.708) (width 0.25) (layer F.Cu) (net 6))
 (segment (start 143.014 76.974) (end 143.28 76.708) (width 0.25) (layer F.Cu) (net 6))
 (segment (start 143.014 77.724) (end 140.97 77.724) (width 0.25) (layer F.Cu) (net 6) (status 10))
 (segment (start 140.474 78.22) (end 140.474 79.756) (width 0.25) (layer F.Cu) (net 6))
 (segment (start 140.97 77.724) (end 140.474 78.22) (width 0.25) (layer F.Cu) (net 6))
 (segment (start 138.418 79.756) (end 140.474 79.756) (width 0.25) (layer F.Cu) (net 6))
 (segment (start 137.481 90.678) (end 135.89 90.678) (width 0.25) (layer F.Cu) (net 6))
 (segment (start 135.382 97.27) (end 135.249 97.403) (width 0.25) (layer F.Cu) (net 6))
 (segment (start 135.249 97.403) (end 134.366 98.286) (width 0.25) (layer F.Cu) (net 6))
 (segment (start 135.382 91.186) (end 135.382 97.27) (width 0.25) (layer F.Cu) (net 6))
 (segment (start 135.89 90.678) (end 135.382 91.186) (width 0.25) (layer F.Cu) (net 6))
 (segment (start 134.354 98.298) (end 134.366 98.286) (width 0.25) (layer F.Cu) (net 6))
 (segment (start 132.854 88.646) (end 132.854 87.872) (width 0.25) (layer F.Cu) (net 7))
 (segment (start 135.433 87.63) (end 137.481 89.678) (width 0.25) (layer F.Cu) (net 7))
 (segment (start 133.096 87.63) (end 135.433 87.63) (width 0.25) (layer F.Cu) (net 7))
 (segment (start 132.854 87.872) (end 133.096 87.63) (width 0.25) (layer F.Cu) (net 7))
 (segment (start 134.354 88.646) (end 134.354 96.774) (width 0.25) (layer F.Cu) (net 8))
 (segment (start 134.354 96.774) (end 134.366 96.786) (width 0.25) (layer F.Cu) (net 8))
 (segment (start 136.93902 83.82) (end 136.93902 79.77702) (width 0.25) (layer F.Cu) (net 9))
 (segment (start 136.93902 79.77702) (end 136.918 79.756) (width 0.25) (layer F.Cu) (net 9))
 (segment (start 141.974 79.756) (end 141.974 83.77498) (width 0.25) (layer F.Cu) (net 10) (status 20))
 (segment (start 141.974 83.77498) (end 142.01902 83.82) (width 0.25) (layer F.Cu) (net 10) (status 30))
 (segment (start 139.946 88.713) (end 139.946 83.84502) (width 0.25) (layer F.Cu) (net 11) (status 20))
 (segment (start 139.946 83.84502) (end 139.92098 83.82) (width 0.25) (layer F.Cu) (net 11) (status 30))
 (segment (start 142.52702 94.742) (end 145.034 94.742) (width 0.25) (layer F.Cu) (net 12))
 (segment (start 146.304 77.724) (end 144.514 77.724) (width 0.25) (layer F.Cu) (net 12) (status 20))
 (via (at 146.304 77.724) (size 0.6) (drill 0.4) (layers F.Cu B.Cu) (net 12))
 (segment (start 146.304 93.472) (end 146.304 77.724) (width 0.25) (layer B.Cu) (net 12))
 (segment (start 145.034 94.742) (end 146.304 93.472) (width 0.25) (layer B.Cu) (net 12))
 (via (at 145.034 94.742) (size 0.6) (drill 0.4) (layers F.Cu B.Cu) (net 12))
 (segment (start 140.42898 94.742) (end 140.42898 92.66002) (width 0.25) (layer F.Cu) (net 13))
 (segment (start 140.42898 92.66002) (end 140.446 92.643) (width 0.25) (layer F.Cu) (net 13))
 (segment (start 148.844 97.79) (end 150.368 97.79) (width 0.25) (layer F.Cu) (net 14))
 (segment (start 155.956 92.202) (end 155.956 90.424) (width 0.25) (layer B.Cu) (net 14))
 (via (at 155.956 92.202) (size 0.6) (drill 0.4) (layers F.Cu B.Cu) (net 14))
 (segment (start 150.368 97.79) (end 155.956 92.202) (width 0.25) (layer F.Cu) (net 14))
 (segment (start 155.956 90.424) (end 156.21 90.424) (width 0.25) (layer B.Cu) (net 14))
 (segment (start 156.21 90.424) (end 158.242 88.392) (width 0.25) (layer B.Cu) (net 14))
 (segment (start 158.242 79.248) (end 156.718 77.724) (width 0.25) (layer F.Cu) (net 14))
 (via (at 158.242 79.248) (size 0.6) (drill 0.4) (layers F.Cu B.Cu) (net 14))
 (segment (start 158.242 88.392) (end 158.242 79.248) (width 0.25) (layer B.Cu) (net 14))
 (segment (start 156.718 77.724) (end 155.956 77.724) (width 0.25) (layer F.Cu) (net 14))
 (segment (start 155.702 90.424) (end 155.956 90.424) (width 0.25) (layer B.Cu) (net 14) (status 30))
 (segment (start 155.956 90.424) (end 156.972 90.424) (width 0.25) (layer B.Cu) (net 14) (status 30))
 (segment (start 138.446 88.713) (end 138.243 88.713) (width 0.25) (layer F.Cu) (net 20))
 (segment (start 153.924 80.264) (end 155.956 80.264) (width 0.25) (layer B.Cu) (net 20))
 (via (at 153.924 80.264) (size 0.6) (drill 0.4) (layers F.Cu B.Cu) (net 20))
 (segment (start 151.892 82.296) (end 153.924 80.264) (width 0.25) (layer F.Cu) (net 20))
 (via (at 151.892 82.296) (size 0.6) (drill 0.4) (layers F.Cu B.Cu) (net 20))
 (segment (start 150.876 83.058) (end 151.892 82.296) (width 0.25) (layer B.Cu) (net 20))
 (segment (start 149.098 84.328) (end 150.876 83.058) (width 0.25) (layer B.Cu) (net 20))
 (via (at 149.098 84.328) (size 0.6) (drill 0.4) (layers F.Cu B.Cu) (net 20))
 (segment (start 146.05 84.328) (end 149.098 84.328) (width 0.25) (layer F.Cu) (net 20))
 (segment (start 144.018 86.36) (end 146.05 84.328) (width 0.25) (layer F.Cu) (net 20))
 (via (at 144.018 86.36) (size 0.6) (drill 0.4) (layers F.Cu B.Cu) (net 20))
 (segment (start 142.748 87.63) (end 144.018 86.36) (width 0.25) (layer B.Cu) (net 20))
 (segment (start 137.16 87.63) (end 142.748 87.63) (width 0.25) (layer B.Cu) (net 20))
 (segment (start 136.906 87.376) (end 137.16 87.63) (width 0.25) (layer B.Cu) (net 20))
 (via (at 136.906 87.376) (size 0.6) (drill 0.4) (layers F.Cu B.Cu) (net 20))
 (segment (start 138.243 88.713) (end 136.906 87.376) (width 0.25) (layer F.Cu) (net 20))
 (segment (start 138.446 88.713) (end 138.446 88.662) (width 0.25) (layer F.Cu) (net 20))
 (segment (start 137.481 91.178) (end 136.406 91.178) (width 0.25) (layer F.Cu) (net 21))
 (segment (start 154.432 82.804) (end 155.956 82.804) (width 0.25) (layer B.Cu) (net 21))
 (segment (start 148.59 76.962) (end 154.432 82.804) (width 0.25) (layer B.Cu) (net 21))
 (segment (start 136.144 76.962) (end 148.59 76.962) (width 0.25) (layer B.Cu) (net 21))
 (segment (start 136.144 91.44) (end 136.144 76.962) (width 0.25) (layer B.Cu) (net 21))
 (via (at 136.144 91.44) (size 0.6) (drill 0.4) (layers F.Cu B.Cu) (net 21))
 (segment (start 136.406 91.178) (end 136.144 91.44) (width 0.25) (layer F.Cu) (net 21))
 (segment (start 149.848 82.55) (end 149.848 84.062) (width 0.25) (layer F.Cu) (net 22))
 (segment (start 153.67 87.884) (end 155.956 87.884) (width 0.25) (layer B.Cu) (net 22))
 (via (at 153.67 87.884) (size 0.6) (drill 0.4) (layers F.Cu B.Cu) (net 22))
 (segment (start 149.848 84.062) (end 153.67 87.884) (width 0.25) (layer F.Cu) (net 22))
 (segment (start 123.06808 79.89316) (end 123.06808 85.39226) (width 0.25) (layer F.Cu) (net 24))
 (segment (start 114.16792 79.89316) (end 123.06808 79.89316) (width 0.25) (layer F.Cu) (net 24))
 (segment (start 114.16792 85.39226) (end 114.16792 79.89316) (width 0.25) (layer F.Cu) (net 24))
 (segment (start 125.972 91.186) (end 125.972 95.492) (width 0.25) (layer F.Cu) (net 25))
 (segment (start 143.784222 91.240096) (end 141.411 91.178) (width 0.25) (layer F.Cu) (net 25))
 (segment (start 143.792222 91.248096) (end 143.784222 91.240096) (width 0.25) (layer F.Cu) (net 25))
 (via (at 143.792222 91.248096) (size 0.6) (drill 0.4) (layers F.Cu B.Cu) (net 25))
 (segment (start 143.764 96.774) (end 143.792222 91.248096) (width 0.25) (layer B.Cu) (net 25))
 (segment (start 142.748 96.774) (end 143.764 96.774) (width 0.25) (layer B.Cu) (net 25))
 (segment (start 127.254 96.774) (end 142.748 96.774) (width 0.25) (layer B.Cu) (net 25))
 (via (at 127.254 96.774) (size 0.6) (drill 0.4) (layers F.Cu B.Cu) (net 25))
 (segment (start 125.972 95.492) (end 127.254 96.774) (width 0.25) (layer F.Cu) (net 25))
 (segment (start 141.411 91.678) (end 142.994435 91.678) (width 0.25) (layer F.Cu) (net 26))
 (segment (start 130.556 93.98) (end 129.528 93.98) (width 0.25) (layer F.Cu) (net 26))
 (segment (start 132.588 96.012) (end 130.556 93.98) (width 0.25) (layer F.Cu) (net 26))
 (via (at 132.588 96.012) (size 0.6) (drill 0.4) (layers F.Cu B.Cu) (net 26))
 (segment (start 143.002 96.012) (end 132.588 96.012) (width 0.25) (layer B.Cu) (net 26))
 (segment (start 143.002 93.218) (end 143.002 96.012) (width 0.25) (layer B.Cu) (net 26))
 (via (at 143.002 93.218) (size 0.6) (drill 0.4) (layers F.Cu B.Cu) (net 26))
 (segment (start 143.002 91.685565) (end 143.002 93.218) (width 0.25) (layer F.Cu) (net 26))
 (segment (start 142.994435 91.678) (end 143.002 91.685565) (width 0.25) (layer F.Cu) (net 26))
 (segment (start 146.062 79.756) (end 145.288 79.756) (width 0.25) (layer F.Cu) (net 27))
 (segment (start 138.946 87.892) (end 138.946 88.713) (width 0.25) (layer F.Cu) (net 27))
 (segment (start 137.922 86.868) (end 138.946 87.892) (width 0.25) (layer F.Cu) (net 27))
 (via (at 137.922 86.868) (size 0.6) (drill 0.4) (layers F.Cu B.Cu) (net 27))
 (segment (start 137.922 82.296) (end 137.922 86.614) (width 0.25) (layer B.Cu) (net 27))
 (segment (start 137.922 82.296) (end 137.922 82.296) (width 0.25) (layer B.Cu) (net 27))
 (segment (start 142.748 82.296) (end 137.922 82.296) (width 0.25) (layer B.Cu) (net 27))
 (segment (start 143.002 82.042) (end 142.748 82.296) (width 0.25) (layer B.Cu) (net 27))
 (via (at 143.002 82.042) (size 0.6) (drill 0.4) (layers F.Cu B.Cu) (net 27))
 (segment (start 145.288 79.756) (end 143.002 82.042) (width 0.25) (layer F.Cu) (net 27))
 (segment (start 139.446 88.713) (end 139.446 87.122) (width 0.25) (layer F.Cu) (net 28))
 (segment (start 144.272 82.55) (end 148.348 82.55) (width 0.25) (layer F.Cu) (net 28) (status 20))
 (segment (start 144.018 82.804) (end 144.272 82.55) (width 0.25) (layer F.Cu) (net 28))
 (via (at 144.018 82.804) (size 0.6) (drill 0.4) (layers F.Cu B.Cu) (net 28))
 (segment (start 144.018 84.836) (end 144.018 82.804) (width 0.25) (layer B.Cu) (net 28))
 (segment (start 142.24 86.614) (end 144.018 84.836) (width 0.25) (layer B.Cu) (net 28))
 (segment (start 139.446 86.614) (end 142.24 86.614) (width 0.25) (layer B.Cu) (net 28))
 (segment (start 139.192 86.868) (end 139.446 86.614) (width 0.25) (layer B.Cu) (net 28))
 (via (at 139.192 86.868) (size 0.6) (drill 0.4) (layers F.Cu B.Cu) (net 28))
 (segment (start 139.446 87.122) (end 139.192 86.868) (width 0.25) (layer F.Cu) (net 28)))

